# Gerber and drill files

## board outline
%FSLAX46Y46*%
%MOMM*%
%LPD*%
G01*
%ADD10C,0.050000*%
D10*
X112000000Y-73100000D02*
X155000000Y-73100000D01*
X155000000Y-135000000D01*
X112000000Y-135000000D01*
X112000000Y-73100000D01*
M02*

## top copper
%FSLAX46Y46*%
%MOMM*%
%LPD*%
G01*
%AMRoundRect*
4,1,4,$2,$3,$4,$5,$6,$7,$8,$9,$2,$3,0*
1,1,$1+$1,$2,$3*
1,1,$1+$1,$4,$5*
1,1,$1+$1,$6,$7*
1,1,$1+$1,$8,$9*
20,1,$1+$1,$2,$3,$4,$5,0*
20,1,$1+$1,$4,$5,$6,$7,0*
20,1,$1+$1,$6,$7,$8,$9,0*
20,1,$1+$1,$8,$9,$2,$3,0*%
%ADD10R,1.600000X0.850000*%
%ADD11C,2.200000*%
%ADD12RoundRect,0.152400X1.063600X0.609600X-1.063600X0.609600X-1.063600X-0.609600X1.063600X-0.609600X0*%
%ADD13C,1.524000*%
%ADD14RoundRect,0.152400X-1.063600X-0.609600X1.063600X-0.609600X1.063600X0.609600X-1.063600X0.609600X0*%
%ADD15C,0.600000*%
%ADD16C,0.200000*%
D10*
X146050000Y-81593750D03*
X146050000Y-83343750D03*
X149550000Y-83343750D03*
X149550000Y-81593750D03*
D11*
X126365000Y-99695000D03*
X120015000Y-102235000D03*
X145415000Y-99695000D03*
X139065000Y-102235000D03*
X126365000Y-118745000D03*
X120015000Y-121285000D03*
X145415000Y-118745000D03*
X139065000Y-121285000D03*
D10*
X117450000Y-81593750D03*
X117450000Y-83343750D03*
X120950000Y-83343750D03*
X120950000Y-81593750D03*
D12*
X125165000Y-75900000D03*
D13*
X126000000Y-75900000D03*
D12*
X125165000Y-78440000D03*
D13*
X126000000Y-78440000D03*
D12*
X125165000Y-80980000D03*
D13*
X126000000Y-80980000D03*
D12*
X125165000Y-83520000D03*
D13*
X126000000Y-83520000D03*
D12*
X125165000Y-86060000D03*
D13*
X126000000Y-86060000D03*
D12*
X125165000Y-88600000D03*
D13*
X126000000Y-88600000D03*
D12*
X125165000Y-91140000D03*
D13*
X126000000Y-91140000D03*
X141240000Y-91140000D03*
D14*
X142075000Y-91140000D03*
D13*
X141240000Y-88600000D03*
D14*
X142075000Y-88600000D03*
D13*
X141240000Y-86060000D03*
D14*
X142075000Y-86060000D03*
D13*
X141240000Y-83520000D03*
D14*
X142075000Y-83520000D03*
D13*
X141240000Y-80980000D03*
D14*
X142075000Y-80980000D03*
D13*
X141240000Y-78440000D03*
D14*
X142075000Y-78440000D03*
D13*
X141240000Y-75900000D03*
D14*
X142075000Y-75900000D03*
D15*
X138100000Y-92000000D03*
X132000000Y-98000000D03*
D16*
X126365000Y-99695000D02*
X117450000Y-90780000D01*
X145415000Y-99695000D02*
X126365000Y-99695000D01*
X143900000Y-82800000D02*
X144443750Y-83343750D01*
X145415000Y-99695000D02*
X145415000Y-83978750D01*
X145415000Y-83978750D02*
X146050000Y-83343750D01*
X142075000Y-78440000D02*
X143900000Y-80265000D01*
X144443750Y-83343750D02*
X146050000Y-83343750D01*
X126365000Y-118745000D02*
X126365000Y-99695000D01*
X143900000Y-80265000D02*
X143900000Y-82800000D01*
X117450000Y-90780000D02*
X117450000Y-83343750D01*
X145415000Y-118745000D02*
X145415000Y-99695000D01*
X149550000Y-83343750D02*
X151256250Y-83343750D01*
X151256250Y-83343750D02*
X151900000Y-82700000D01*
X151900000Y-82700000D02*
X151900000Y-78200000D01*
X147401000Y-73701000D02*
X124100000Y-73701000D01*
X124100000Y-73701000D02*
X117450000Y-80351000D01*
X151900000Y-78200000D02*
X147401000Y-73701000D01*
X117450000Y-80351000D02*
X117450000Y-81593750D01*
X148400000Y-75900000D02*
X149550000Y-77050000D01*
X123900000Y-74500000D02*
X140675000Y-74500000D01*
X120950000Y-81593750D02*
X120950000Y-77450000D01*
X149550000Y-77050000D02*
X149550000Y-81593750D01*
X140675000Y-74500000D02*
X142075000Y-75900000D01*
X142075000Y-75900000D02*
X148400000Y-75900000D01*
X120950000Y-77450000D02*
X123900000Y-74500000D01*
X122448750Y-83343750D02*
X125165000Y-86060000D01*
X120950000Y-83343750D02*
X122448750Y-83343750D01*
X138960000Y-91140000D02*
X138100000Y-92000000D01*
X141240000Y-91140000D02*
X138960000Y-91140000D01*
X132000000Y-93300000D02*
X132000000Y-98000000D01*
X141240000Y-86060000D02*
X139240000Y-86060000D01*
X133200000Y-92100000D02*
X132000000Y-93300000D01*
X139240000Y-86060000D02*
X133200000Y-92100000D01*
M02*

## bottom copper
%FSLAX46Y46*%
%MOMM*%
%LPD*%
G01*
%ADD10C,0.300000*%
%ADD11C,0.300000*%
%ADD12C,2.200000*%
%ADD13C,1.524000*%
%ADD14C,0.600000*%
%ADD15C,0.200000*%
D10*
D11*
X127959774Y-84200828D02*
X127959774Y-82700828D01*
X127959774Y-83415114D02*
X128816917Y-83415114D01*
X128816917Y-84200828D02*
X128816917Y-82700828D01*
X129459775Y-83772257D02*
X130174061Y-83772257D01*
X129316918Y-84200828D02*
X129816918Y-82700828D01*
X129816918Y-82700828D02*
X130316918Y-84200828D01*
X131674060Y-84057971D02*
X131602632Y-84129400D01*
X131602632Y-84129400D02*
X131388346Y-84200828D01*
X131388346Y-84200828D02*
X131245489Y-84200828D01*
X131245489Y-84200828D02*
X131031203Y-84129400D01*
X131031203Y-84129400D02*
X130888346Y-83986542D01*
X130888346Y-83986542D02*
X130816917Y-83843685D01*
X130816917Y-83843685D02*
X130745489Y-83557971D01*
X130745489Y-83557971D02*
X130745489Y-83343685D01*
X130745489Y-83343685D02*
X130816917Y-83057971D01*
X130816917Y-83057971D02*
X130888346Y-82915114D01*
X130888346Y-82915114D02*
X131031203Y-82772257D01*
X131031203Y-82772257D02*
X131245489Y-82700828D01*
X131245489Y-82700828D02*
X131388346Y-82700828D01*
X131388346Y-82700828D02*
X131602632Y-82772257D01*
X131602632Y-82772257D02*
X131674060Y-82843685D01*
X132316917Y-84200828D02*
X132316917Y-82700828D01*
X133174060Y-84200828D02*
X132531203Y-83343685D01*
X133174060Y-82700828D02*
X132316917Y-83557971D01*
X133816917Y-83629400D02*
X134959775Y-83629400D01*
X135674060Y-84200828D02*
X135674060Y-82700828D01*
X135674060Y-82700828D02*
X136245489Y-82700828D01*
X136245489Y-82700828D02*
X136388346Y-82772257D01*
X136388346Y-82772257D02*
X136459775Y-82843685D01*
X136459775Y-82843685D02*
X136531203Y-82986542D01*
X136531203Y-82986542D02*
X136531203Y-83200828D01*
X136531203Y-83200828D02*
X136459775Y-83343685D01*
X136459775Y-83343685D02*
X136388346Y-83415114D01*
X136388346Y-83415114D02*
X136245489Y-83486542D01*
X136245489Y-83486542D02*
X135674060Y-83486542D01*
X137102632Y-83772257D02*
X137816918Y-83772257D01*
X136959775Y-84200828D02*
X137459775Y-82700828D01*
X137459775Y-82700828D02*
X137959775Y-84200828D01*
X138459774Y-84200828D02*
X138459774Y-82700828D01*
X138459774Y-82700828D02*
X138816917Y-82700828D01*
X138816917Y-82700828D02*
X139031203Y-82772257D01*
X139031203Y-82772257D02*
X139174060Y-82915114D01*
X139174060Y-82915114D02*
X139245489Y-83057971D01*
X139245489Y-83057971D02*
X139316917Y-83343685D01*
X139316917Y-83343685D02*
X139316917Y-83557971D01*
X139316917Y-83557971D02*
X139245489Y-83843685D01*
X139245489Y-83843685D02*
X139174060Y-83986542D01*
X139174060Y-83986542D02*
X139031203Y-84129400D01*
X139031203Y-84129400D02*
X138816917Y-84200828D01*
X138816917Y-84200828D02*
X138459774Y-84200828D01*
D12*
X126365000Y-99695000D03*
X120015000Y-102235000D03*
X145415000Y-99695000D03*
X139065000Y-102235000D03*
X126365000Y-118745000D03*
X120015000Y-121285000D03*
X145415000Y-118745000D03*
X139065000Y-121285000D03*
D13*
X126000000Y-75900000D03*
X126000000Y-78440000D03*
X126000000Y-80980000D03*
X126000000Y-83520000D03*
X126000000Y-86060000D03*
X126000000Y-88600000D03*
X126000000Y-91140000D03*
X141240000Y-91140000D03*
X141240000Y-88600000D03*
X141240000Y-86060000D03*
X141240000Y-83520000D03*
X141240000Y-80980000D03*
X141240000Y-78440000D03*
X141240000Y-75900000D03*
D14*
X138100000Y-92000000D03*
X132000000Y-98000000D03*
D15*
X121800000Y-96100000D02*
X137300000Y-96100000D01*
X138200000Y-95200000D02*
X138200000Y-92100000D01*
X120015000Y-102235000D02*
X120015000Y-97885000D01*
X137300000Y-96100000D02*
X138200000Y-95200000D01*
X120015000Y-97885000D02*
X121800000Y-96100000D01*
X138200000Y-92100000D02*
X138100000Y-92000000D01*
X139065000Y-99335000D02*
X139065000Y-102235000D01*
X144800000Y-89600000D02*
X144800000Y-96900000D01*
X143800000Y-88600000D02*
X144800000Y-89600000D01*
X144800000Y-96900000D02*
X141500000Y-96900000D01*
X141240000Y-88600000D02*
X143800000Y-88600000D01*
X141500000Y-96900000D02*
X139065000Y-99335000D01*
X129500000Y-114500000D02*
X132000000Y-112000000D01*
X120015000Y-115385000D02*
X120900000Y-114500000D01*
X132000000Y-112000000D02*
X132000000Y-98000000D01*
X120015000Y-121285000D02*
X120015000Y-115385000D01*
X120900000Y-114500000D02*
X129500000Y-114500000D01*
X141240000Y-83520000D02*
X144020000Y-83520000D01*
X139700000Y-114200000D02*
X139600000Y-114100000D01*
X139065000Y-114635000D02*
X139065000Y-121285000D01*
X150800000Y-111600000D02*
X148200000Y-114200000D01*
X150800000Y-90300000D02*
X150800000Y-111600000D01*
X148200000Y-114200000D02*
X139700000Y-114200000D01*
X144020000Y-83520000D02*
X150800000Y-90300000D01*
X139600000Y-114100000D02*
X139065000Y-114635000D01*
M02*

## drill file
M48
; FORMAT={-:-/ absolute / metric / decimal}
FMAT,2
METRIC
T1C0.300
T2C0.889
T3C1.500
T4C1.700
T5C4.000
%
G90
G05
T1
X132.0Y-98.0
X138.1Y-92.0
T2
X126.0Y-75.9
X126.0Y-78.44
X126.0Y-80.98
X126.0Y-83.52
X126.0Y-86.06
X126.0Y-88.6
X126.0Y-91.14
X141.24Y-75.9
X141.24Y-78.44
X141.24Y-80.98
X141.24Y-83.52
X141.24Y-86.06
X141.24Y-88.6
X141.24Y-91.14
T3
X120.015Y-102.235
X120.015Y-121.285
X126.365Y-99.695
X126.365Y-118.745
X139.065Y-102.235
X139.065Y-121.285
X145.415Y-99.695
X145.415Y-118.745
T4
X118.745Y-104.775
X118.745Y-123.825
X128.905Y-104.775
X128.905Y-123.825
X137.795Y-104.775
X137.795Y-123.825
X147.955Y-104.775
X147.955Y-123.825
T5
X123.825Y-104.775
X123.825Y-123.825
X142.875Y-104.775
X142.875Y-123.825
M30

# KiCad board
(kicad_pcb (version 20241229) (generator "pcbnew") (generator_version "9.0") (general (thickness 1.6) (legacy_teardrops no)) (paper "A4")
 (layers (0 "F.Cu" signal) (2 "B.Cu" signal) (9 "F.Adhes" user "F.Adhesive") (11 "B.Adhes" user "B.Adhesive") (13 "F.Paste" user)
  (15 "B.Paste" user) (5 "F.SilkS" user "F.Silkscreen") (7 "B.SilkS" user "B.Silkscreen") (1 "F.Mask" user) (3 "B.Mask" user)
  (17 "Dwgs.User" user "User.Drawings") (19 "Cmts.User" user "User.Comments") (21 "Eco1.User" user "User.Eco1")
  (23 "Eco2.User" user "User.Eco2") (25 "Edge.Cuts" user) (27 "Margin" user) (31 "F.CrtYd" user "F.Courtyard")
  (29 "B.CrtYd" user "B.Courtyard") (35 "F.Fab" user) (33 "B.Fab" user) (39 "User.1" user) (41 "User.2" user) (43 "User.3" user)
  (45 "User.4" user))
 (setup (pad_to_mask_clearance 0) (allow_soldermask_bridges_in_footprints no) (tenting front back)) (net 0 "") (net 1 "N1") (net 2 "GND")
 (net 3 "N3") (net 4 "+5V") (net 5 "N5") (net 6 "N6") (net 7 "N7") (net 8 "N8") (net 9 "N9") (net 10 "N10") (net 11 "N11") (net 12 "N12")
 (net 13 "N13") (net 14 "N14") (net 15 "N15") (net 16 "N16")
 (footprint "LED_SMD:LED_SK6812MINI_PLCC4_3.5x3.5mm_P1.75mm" (layer "F.Cu") (at 147.8 82.46875)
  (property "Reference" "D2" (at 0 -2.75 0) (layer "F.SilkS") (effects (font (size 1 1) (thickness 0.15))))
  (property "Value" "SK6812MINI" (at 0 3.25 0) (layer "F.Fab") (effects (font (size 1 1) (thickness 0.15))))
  (pad "1" smd rect (at -1.75 -0.875) (size 1.6 0.85) (layers "F.Cu" "F.Mask" "F.Paste") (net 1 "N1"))
  (pad "2" smd rect (at -1.75 0.875) (size 1.6 0.85) (layers "F.Cu" "F.Mask" "F.Paste") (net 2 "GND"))
  (pad "3" smd rect (at 1.75 0.875) (size 1.6 0.85) (layers "F.Cu" "F.Mask" "F.Paste") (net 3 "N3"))
  (pad "4" smd rect (at 1.75 -0.875) (size 1.6 0.85) (layers "F.Cu" "F.Mask" "F.Paste") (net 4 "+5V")))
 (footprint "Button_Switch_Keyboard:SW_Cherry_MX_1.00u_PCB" (layer "F.Cu") (at 126.365 99.695)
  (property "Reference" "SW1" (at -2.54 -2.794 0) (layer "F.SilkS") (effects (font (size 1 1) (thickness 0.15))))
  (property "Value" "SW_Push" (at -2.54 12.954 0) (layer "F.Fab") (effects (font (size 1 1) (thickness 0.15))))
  (pad "" np_thru_hole circle (at -7.62 5.08) (size 1.7 1.7) (drill 1.7) (layers "*.Cu" "*.Mask"))
  (pad "" np_thru_hole circle (at -2.54 5.08) (size 4 4) (drill 4) (layers "*.Cu" "*.Mask"))
  (pad "" np_thru_hole circle (at 2.54 5.08) (size 1.7 1.7) (drill 1.7) (layers "*.Cu" "*.Mask"))
  (pad "1" thru_hole circle (at 0 0) (size 2.2 2.2) (drill 1.5) (layers "*.Cu" "*.Mask") (remove_unused_layers no) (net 2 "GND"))
  (pad "2" thru_hole circle (at -6.35 2.54) (size 2.2 2.2) (drill 1.5) (layers "*.Cu" "*.Mask") (remove_unused_layers no) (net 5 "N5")))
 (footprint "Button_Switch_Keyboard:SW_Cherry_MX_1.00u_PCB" (layer "F.Cu") (at 145.415 99.695)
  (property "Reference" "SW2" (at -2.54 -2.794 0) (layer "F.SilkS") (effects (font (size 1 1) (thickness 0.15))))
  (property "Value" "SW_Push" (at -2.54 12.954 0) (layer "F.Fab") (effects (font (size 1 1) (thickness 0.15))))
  (pad "" np_thru_hole circle (at -7.62 5.08) (size 1.7 1.7) (drill 1.7) (layers "*.Cu" "*.Mask"))
  (pad "" np_thru_hole circle (at -2.54 5.08) (size 4 4) (drill 4) (layers "*.Cu" "*.Mask"))
  (pad "" np_thru_hole circle (at 2.54 5.08) (size 1.7 1.7) (drill 1.7) (layers "*.Cu" "*.Mask"))
  (pad "1" thru_hole circle (at 0 0) (size 2.2 2.2) (drill 1.5) (layers "*.Cu" "*.Mask") (remove_unused_layers no) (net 2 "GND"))
  (pad "2" thru_hole circle (at -6.35 2.54) (size 2.2 2.2) (drill 1.5) (layers "*.Cu" "*.Mask") (remove_unused_layers no) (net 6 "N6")))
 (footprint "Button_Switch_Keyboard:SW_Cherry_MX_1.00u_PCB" (layer "F.Cu") (at 126.365 118.745)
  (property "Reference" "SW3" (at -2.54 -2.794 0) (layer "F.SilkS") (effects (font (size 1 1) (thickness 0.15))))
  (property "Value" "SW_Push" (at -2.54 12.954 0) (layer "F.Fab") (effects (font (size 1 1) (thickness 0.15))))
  (pad "" np_thru_hole circle (at -7.62 5.08) (size 1.7 1.7) (drill 1.7) (layers "*.Cu" "*.Mask"))
  (pad "" np_thru_hole circle (at -2.54 5.08) (size 4 4) (drill 4) (layers "*.Cu" "*.Mask"))
  (pad "" np_thru_hole circle (at 2.54 5.08) (size 1.7 1.7) (drill 1.7) (layers "*.Cu" "*.Mask"))
  (pad "1" thru_hole circle (at 0 0) (size 2.2 2.2) (drill 1.5) (layers "*.Cu" "*.Mask") (remove_unused_layers no) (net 2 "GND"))
  (pad "2" thru_hole circle (at -6.35 2.54) (size 2.2 2.2) (drill 1.5) (layers "*.Cu" "*.Mask") (remove_unused_layers no) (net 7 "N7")))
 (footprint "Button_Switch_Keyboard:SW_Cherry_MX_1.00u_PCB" (layer "F.Cu") (at 145.415 118.745)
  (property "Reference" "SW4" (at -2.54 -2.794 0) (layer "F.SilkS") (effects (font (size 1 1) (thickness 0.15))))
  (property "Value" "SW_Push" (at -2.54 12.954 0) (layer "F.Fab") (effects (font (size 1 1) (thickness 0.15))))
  (pad "" np_thru_hole circle (at -7.62 5.08) (size 1.7 1.7) (drill 1.7) (layers "*.Cu" "*.Mask"))
  (pad "" np_thru_hole circle (at -2.54 5.08) (size 4 4) (drill 4) (layers "*.Cu" "*.Mask"))
  (pad "" np_thru_hole circle (at 2.54 5.08) (size 1.7 1.7) (drill 1.7) (layers "*.Cu" "*.Mask"))
  (pad "1" thru_hole circle (at 0 0) (size 2.2 2.2) (drill 1.5) (layers "*.Cu" "*.Mask") (remove_unused_layers no) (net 2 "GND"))
  (pad "2" thru_hole circle (at -6.35 2.54) (size 2.2 2.2) (drill 1.5) (layers "*.Cu" "*.Mask") (remove_unused_layers no) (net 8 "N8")))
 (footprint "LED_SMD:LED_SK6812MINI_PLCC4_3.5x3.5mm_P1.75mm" (layer "F.Cu") (at 119.2 82.46875)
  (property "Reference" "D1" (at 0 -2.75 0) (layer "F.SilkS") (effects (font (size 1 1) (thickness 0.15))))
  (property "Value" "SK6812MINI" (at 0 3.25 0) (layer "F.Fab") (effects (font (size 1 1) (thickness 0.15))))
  (pad "1" smd rect (at -1.75 -0.875) (size 1.6 0.85) (layers "F.Cu" "F.Mask" "F.Paste") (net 3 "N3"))
  (pad "2" smd rect (at -1.75 0.875) (size 1.6 0.85) (layers "F.Cu" "F.Mask" "F.Paste") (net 2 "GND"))
  (pad "3" smd rect (at 1.75 0.875) (size 1.6 0.85) (layers "F.Cu" "F.Mask" "F.Paste") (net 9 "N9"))
  (pad "4" smd rect (at 1.75 -0.875) (size 1.6 0.85) (layers "F.Cu" "F.Mask" "F.Paste") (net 4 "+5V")))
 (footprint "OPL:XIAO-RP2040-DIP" (layer "F.Cu") (at 133.62 83.52)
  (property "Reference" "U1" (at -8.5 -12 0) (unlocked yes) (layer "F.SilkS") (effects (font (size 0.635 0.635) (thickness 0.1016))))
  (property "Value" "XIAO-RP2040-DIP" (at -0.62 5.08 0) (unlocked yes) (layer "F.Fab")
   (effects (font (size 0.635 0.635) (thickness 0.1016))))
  (pad "1" smd roundrect (at -8.455 -7.62 180) (size 2.432 1.524) (layers "F.Cu" "F.Mask") (roundrect_rratio 0.1) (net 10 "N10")
   (thermal_bridge_angle 45))
  (pad "1" thru_hole circle (at -7.62 -7.62 180) (size 1.524 1.524) (drill 0.889) (layers "*.Cu" "*.Mask") (remove_unused_layers no)
   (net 10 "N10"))
  (pad "2" smd roundrect (at -8.455 -5.08 180) (size 2.432 1.524) (layers "F.Cu" "F.Mask") (roundrect_rratio 0.1) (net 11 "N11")
   (thermal_bridge_angle 45))
  (pad "2" thru_hole circle (at -7.62 -5.08 180) (size 1.524 1.524) (drill 0.889) (layers "*.Cu" "*.Mask") (remove_unused_layers no)
   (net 11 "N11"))
  (pad "3" smd roundrect (at -8.455 -2.54 180) (size 2.432 1.524) (layers "F.Cu" "F.Mask") (roundrect_rratio 0.1) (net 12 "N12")
   (thermal_bridge_angle 45))
  (pad "3" thru_hole circle (at -7.62 -2.54 180) (size 1.524 1.524) (drill 0.889) (layers "*.Cu" "*.Mask") (remove_unused_layers no)
   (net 12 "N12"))
  (pad "4" smd roundrect (at -8.455 0 180) (size 2.432 1.524) (layers "F.Cu" "F.Mask") (roundrect_rratio 0.1) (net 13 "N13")
   (thermal_bridge_angle 45))
  (pad "4" thru_hole circle (at -7.62 0 180) (size 1.524 1.524) (drill 0.889) (layers "*.Cu" "*.Mask") (remove_unused_layers no)
   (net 13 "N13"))
  (pad "5" smd roundrect (at -8.455 2.54 180) (size 2.432 1.524) (layers "F.Cu" "F.Mask") (roundrect_rratio 0.1) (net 9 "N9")
   (thermal_bridge_angle 45))
  (pad "5" thru_hole circle (at -7.62 2.54 180) (size 1.524 1.524) (drill 0.889) (layers "*.Cu" "*.Mask") (remove_unused_layers no)
   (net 9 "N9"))
  (pad "6" smd roundrect (at -8.455 5.08 180) (size 2.432 1.524) (layers "F.Cu" "F.Mask") (roundrect_rratio 0.1) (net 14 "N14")
   (thermal_bridge_angle 45))
  (pad "6" thru_hole circle (at -7.62 5.08 180) (size 1.524 1.524) (drill 0.889) (layers "*.Cu" "*.Mask") (remove_unused_layers no)
   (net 14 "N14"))
  (pad "7" smd roundrect (at -8.455 7.62 180) (size 2.432 1.524) (layers "F.Cu" "F.Mask") (roundrect_rratio 0.1) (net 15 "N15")
   (thermal_bridge_angle 45))
  (pad "7" thru_hole circle (at -7.62 7.62 180) (size 1.524 1.524) (drill 0.889) (layers "*.Cu" "*.Mask") (remove_unused_layers no)
   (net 15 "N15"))
  (pad "8" thru_hole circle (at 7.62 7.62) (size 1.524 1.524) (drill 0.889) (layers "*.Cu" "*.Mask") (remove_unused_layers no) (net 5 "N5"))
  (pad "8" smd roundrect (at 8.455 7.62) (size 2.432 1.524) (layers "F.Cu" "F.Mask") (roundrect_rratio 0.1) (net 5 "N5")
   (thermal_bridge_angle 45))
  (pad "9" thru_hole circle (at 7.62 5.08) (size 1.524 1.524) (drill 0.889) (layers "*.Cu" "*.Mask") (remove_unused_layers no) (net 6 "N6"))
  (pad "9" smd roundrect (at 8.455 5.08) (size 2.432 1.524) (layers "F.Cu" "F.Mask") (roundrect_rratio 0.1) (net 6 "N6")
   (thermal_bridge_angle 45))
  (pad "10" thru_hole circle (at 7.62 2.54) (size 1.524 1.524) (drill 0.889) (layers "*.Cu" "*.Mask") (remove_unused_layers no) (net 7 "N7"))
  (pad "10" smd roundrect (at 8.455 2.54) (size 2.432 1.524) (layers "F.Cu" "F.Mask") (roundrect_rratio 0.1) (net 7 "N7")
   (thermal_bridge_angle 45))
  (pad "11" thru_hole circle (at 7.62 0) (size 1.524 1.524) (drill 0.889) (layers "*.Cu" "*.Mask") (remove_unused_layers no) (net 8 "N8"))
  (pad "11" smd roundrect (at 8.455 0) (size 2.432 1.524) (layers "F.Cu" "F.Mask") (roundrect_rratio 0.1) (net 8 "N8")
   (thermal_bridge_angle 45))
  (pad "12" thru_hole circle (at 7.62 -2.54) (size 1.524 1.524) (drill 0.889) (layers "*.Cu" "*.Mask") (remove_unused_layers no)
   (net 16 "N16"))
  (pad "12" smd roundrect (at 8.455 -2.54) (size 2.432 1.524) (layers "F.Cu" "F.Mask") (roundrect_rratio 0.1) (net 16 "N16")
   (thermal_bridge_angle 45))
  (pad "13" thru_hole circle (at 7.62 -5.08) (size 1.524 1.524) (drill 0.889) (layers "*.Cu" "*.Mask") (remove_unused_layers no)
   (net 2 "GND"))
  (pad "13" smd roundrect (at 8.455 -5.08) (size 2.432 1.524) (layers "F.Cu" "F.Mask") (roundrect_rratio 0.1) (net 2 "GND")
   (thermal_bridge_angle 45))
  (pad "14" thru_hole circle (at 7.62 -7.62) (size 1.524 1.524) (drill 0.889) (layers "*.Cu" "*.Mask") (remove_unused_layers no)
   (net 4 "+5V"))
  (pad "14" smd roundrect (at 8.455 -7.62) (size 2.432 1.524) (layers "F.Cu" "F.Mask") (roundrect_rratio 0.1) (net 4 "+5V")
   (thermal_bridge_angle 45)))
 (gr_rect (start 112 73.1) (end 155 135) (stroke (width 0.05) (type default)) (fill no) (layer "Edge.Cuts"))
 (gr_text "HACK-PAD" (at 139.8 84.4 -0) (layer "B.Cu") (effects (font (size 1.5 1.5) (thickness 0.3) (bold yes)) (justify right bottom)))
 (segment (start 126.365 99.695) (end 117.45 90.78) (width 0.2) (layer "F.Cu") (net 2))
 (segment (start 145.415 99.695) (end 126.365 99.695) (width 0.2) (layer "F.Cu") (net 2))
 (segment (start 143.9 82.8) (end 144.44375 83.34375) (width 0.2) (layer "F.Cu") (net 2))
 (segment (start 145.415 99.695) (end 145.415 83.97875) (width 0.2) (layer "F.Cu") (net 2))
 (segment (start 145.415 83.97875) (end 146.05 83.34375) (width 0.2) (layer "F.Cu") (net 2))
 (segment (start 142.075 78.44) (end 143.9 80.265) (width 0.2) (layer "F.Cu") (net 2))
 (segment (start 144.44375 83.34375) (end 146.05 83.34375) (width 0.2) (layer "F.Cu") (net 2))
 (segment (start 126.365 118.745) (end 126.365 99.695) (width 0.2) (layer "F.Cu") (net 2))
 (segment (start 143.9 80.265) (end 143.9 82.8) (width 0.2) (layer "F.Cu") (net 2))
 (segment (start 117.45 90.78) (end 117.45 83.34375) (width 0.2) (layer "F.Cu") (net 2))
 (segment (start 145.415 118.745) (end 145.415 99.695) (width 0.2) (layer "F.Cu") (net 2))
 (segment (start 149.55 83.34375) (end 151.25625 83.34375) (width 0.2) (layer "F.Cu") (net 3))
 (segment (start 151.25625 83.34375) (end 151.9 82.7) (width 0.2) (layer "F.Cu") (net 3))
 (segment (start 151.9 82.7) (end 151.9 78.2) (width 0.2) (layer "F.Cu") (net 3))
 (segment (start 147.401 73.701) (end 124.1 73.701) (width 0.2) (layer "F.Cu") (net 3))
 (segment (start 124.1 73.701) (end 117.45 80.351) (width 0.2) (layer "F.Cu") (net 3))
 (segment (start 151.9 78.2) (end 147.401 73.701) (width 0.2) (layer "F.Cu") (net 3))
 (segment (start 117.45 80.351) (end 117.45 81.59375) (width 0.2) (layer "F.Cu") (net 3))
 (segment (start 148.4 75.9) (end 149.55 77.05) (width 0.2) (layer "F.Cu") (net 4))
 (segment (start 123.9 74.5) (end 140.675 74.5) (width 0.2) (layer "F.Cu") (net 4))
 (segment (start 120.95 81.59375) (end 120.95 77.45) (width 0.2) (layer "F.Cu") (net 4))
 (segment (start 149.55 77.05) (end 149.55 81.59375) (width 0.2) (layer "F.Cu") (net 4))
 (segment (start 140.675 74.5) (end 142.075 75.9) (width 0.2) (layer "F.Cu") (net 4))
 (segment (start 142.075 75.9) (end 148.4 75.9) (width 0.2) (layer "F.Cu") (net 4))
 (segment (start 120.95 77.45) (end 123.9 74.5) (width 0.2) (layer "F.Cu") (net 4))
 (segment (start 122.44875 83.34375) (end 125.165 86.06) (width 0.2) (layer "F.Cu") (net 9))
 (segment (start 120.95 83.34375) (end 122.44875 83.34375) (width 0.2) (layer "F.Cu") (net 9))
 (segment (start 138.96 91.14) (end 138.1 92) (width 0.2) (layer "F.Cu") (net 5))
 (segment (start 141.24 91.14) (end 138.96 91.14) (width 0.2) (layer "F.Cu") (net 5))
 (via (at 138.1 92) (size 0.6) (drill 0.3) (layers "F.Cu" "B.Cu") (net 5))
 (segment (start 121.8 96.1) (end 137.3 96.1) (width 0.2) (layer "B.Cu") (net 5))
 (segment (start 138.2 95.2) (end 138.2 92.1) (width 0.2) (layer "B.Cu") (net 5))
 (segment (start 120.015 102.235) (end 120.015 97.885) (width 0.2) (layer "B.Cu") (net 5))
 (segment (start 137.3 96.1) (end 138.2 95.2) (width 0.2) (layer "B.Cu") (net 5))
 (segment (start 120.015 97.885) (end 121.8 96.1) (width 0.2) (layer "B.Cu") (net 5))
 (segment (start 138.2 92.1) (end 138.1 92) (width 0.2) (layer "B.Cu") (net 5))
 (segment (start 139.065 99.335) (end 139.065 102.235) (width 0.2) (layer "B.Cu") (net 6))
 (segment (start 144.8 89.6) (end 144.8 96.9) (width 0.2) (layer "B.Cu") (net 6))
 (segment (start 143.8 88.6) (end 144.8 89.6) (width 0.2) (layer "B.Cu") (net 6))
 (segment (start 144.8 96.9) (end 141.5 96.9) (width 0.2) (layer "B.Cu") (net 6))
 (segment (start 141.24 88.6) (end 143.8 88.6) (width 0.2) (layer "B.Cu") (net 6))
 (segment (start 141.5 96.9) (end 139.065 99.335) (width 0.2) (layer "B.Cu") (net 6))
 (segment (start 132 93.3) (end 132 98) (width 0.2) (layer "F.Cu") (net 7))
 (segment (start 141.24 86.06) (end 139.24 86.06) (width 0.2) (layer "F.Cu") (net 7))
 (segment (start 133.2 92.1) (end 132 93.3) (width 0.2) (layer "F.Cu") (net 7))
 (segment (start 139.24 86.06) (end 133.2 92.1) (width 0.2) (layer "F.Cu") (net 7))
 (via (at 132 98) (size 0.6) (drill 0.3) (layers "F.Cu" "B.Cu") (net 7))
 (segment (start 129.5 114.5) (end 132 112) (width 0.2) (layer "B.Cu") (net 7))
 (segment (start 120.015 115.385) (end 120.9 114.5) (width 0.2) (layer "B.Cu") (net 7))
 (segment (start 132 112) (end 132 98) (width 0.2) (layer "B.Cu") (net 7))
 (segment (start 120.015 121.285) (end 120.015 115.385) (width 0.2) (layer "B.Cu") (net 7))
 (segment (start 120.9 114.5) (end 129.5 114.5) (width 0.2) (layer "B.Cu") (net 7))
 (segment (start 141.24 83.52) (end 144.02 83.52) (width 0.2) (layer "B.Cu") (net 8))
 (segment (start 139.7 114.2) (end 139.6 114.1) (width 0.2) (layer "B.Cu") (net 8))
 (segment (start 139.065 114.635) (end 139.065 121.285) (width 0.2) (layer "B.Cu") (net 8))
 (segment (start 150.8 111.6) (end 148.2 114.2) (width 0.2) (layer "B.Cu") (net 8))
 (segment (start 150.8 90.3) (end 150.8 111.6) (width 0.2) (layer "B.Cu") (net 8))
 (segment (start 148.2 114.2) (end 139.7 114.2) (width 0.2) (layer "B.Cu") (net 8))
 (segment (start 144.02 83.52) (end 150.8 90.3) (width 0.2) (layer "B.Cu") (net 8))
 (segment (start 139.6 114.1) (end 139.065 114.635) (width 0.2) (layer "B.Cu") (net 8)))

